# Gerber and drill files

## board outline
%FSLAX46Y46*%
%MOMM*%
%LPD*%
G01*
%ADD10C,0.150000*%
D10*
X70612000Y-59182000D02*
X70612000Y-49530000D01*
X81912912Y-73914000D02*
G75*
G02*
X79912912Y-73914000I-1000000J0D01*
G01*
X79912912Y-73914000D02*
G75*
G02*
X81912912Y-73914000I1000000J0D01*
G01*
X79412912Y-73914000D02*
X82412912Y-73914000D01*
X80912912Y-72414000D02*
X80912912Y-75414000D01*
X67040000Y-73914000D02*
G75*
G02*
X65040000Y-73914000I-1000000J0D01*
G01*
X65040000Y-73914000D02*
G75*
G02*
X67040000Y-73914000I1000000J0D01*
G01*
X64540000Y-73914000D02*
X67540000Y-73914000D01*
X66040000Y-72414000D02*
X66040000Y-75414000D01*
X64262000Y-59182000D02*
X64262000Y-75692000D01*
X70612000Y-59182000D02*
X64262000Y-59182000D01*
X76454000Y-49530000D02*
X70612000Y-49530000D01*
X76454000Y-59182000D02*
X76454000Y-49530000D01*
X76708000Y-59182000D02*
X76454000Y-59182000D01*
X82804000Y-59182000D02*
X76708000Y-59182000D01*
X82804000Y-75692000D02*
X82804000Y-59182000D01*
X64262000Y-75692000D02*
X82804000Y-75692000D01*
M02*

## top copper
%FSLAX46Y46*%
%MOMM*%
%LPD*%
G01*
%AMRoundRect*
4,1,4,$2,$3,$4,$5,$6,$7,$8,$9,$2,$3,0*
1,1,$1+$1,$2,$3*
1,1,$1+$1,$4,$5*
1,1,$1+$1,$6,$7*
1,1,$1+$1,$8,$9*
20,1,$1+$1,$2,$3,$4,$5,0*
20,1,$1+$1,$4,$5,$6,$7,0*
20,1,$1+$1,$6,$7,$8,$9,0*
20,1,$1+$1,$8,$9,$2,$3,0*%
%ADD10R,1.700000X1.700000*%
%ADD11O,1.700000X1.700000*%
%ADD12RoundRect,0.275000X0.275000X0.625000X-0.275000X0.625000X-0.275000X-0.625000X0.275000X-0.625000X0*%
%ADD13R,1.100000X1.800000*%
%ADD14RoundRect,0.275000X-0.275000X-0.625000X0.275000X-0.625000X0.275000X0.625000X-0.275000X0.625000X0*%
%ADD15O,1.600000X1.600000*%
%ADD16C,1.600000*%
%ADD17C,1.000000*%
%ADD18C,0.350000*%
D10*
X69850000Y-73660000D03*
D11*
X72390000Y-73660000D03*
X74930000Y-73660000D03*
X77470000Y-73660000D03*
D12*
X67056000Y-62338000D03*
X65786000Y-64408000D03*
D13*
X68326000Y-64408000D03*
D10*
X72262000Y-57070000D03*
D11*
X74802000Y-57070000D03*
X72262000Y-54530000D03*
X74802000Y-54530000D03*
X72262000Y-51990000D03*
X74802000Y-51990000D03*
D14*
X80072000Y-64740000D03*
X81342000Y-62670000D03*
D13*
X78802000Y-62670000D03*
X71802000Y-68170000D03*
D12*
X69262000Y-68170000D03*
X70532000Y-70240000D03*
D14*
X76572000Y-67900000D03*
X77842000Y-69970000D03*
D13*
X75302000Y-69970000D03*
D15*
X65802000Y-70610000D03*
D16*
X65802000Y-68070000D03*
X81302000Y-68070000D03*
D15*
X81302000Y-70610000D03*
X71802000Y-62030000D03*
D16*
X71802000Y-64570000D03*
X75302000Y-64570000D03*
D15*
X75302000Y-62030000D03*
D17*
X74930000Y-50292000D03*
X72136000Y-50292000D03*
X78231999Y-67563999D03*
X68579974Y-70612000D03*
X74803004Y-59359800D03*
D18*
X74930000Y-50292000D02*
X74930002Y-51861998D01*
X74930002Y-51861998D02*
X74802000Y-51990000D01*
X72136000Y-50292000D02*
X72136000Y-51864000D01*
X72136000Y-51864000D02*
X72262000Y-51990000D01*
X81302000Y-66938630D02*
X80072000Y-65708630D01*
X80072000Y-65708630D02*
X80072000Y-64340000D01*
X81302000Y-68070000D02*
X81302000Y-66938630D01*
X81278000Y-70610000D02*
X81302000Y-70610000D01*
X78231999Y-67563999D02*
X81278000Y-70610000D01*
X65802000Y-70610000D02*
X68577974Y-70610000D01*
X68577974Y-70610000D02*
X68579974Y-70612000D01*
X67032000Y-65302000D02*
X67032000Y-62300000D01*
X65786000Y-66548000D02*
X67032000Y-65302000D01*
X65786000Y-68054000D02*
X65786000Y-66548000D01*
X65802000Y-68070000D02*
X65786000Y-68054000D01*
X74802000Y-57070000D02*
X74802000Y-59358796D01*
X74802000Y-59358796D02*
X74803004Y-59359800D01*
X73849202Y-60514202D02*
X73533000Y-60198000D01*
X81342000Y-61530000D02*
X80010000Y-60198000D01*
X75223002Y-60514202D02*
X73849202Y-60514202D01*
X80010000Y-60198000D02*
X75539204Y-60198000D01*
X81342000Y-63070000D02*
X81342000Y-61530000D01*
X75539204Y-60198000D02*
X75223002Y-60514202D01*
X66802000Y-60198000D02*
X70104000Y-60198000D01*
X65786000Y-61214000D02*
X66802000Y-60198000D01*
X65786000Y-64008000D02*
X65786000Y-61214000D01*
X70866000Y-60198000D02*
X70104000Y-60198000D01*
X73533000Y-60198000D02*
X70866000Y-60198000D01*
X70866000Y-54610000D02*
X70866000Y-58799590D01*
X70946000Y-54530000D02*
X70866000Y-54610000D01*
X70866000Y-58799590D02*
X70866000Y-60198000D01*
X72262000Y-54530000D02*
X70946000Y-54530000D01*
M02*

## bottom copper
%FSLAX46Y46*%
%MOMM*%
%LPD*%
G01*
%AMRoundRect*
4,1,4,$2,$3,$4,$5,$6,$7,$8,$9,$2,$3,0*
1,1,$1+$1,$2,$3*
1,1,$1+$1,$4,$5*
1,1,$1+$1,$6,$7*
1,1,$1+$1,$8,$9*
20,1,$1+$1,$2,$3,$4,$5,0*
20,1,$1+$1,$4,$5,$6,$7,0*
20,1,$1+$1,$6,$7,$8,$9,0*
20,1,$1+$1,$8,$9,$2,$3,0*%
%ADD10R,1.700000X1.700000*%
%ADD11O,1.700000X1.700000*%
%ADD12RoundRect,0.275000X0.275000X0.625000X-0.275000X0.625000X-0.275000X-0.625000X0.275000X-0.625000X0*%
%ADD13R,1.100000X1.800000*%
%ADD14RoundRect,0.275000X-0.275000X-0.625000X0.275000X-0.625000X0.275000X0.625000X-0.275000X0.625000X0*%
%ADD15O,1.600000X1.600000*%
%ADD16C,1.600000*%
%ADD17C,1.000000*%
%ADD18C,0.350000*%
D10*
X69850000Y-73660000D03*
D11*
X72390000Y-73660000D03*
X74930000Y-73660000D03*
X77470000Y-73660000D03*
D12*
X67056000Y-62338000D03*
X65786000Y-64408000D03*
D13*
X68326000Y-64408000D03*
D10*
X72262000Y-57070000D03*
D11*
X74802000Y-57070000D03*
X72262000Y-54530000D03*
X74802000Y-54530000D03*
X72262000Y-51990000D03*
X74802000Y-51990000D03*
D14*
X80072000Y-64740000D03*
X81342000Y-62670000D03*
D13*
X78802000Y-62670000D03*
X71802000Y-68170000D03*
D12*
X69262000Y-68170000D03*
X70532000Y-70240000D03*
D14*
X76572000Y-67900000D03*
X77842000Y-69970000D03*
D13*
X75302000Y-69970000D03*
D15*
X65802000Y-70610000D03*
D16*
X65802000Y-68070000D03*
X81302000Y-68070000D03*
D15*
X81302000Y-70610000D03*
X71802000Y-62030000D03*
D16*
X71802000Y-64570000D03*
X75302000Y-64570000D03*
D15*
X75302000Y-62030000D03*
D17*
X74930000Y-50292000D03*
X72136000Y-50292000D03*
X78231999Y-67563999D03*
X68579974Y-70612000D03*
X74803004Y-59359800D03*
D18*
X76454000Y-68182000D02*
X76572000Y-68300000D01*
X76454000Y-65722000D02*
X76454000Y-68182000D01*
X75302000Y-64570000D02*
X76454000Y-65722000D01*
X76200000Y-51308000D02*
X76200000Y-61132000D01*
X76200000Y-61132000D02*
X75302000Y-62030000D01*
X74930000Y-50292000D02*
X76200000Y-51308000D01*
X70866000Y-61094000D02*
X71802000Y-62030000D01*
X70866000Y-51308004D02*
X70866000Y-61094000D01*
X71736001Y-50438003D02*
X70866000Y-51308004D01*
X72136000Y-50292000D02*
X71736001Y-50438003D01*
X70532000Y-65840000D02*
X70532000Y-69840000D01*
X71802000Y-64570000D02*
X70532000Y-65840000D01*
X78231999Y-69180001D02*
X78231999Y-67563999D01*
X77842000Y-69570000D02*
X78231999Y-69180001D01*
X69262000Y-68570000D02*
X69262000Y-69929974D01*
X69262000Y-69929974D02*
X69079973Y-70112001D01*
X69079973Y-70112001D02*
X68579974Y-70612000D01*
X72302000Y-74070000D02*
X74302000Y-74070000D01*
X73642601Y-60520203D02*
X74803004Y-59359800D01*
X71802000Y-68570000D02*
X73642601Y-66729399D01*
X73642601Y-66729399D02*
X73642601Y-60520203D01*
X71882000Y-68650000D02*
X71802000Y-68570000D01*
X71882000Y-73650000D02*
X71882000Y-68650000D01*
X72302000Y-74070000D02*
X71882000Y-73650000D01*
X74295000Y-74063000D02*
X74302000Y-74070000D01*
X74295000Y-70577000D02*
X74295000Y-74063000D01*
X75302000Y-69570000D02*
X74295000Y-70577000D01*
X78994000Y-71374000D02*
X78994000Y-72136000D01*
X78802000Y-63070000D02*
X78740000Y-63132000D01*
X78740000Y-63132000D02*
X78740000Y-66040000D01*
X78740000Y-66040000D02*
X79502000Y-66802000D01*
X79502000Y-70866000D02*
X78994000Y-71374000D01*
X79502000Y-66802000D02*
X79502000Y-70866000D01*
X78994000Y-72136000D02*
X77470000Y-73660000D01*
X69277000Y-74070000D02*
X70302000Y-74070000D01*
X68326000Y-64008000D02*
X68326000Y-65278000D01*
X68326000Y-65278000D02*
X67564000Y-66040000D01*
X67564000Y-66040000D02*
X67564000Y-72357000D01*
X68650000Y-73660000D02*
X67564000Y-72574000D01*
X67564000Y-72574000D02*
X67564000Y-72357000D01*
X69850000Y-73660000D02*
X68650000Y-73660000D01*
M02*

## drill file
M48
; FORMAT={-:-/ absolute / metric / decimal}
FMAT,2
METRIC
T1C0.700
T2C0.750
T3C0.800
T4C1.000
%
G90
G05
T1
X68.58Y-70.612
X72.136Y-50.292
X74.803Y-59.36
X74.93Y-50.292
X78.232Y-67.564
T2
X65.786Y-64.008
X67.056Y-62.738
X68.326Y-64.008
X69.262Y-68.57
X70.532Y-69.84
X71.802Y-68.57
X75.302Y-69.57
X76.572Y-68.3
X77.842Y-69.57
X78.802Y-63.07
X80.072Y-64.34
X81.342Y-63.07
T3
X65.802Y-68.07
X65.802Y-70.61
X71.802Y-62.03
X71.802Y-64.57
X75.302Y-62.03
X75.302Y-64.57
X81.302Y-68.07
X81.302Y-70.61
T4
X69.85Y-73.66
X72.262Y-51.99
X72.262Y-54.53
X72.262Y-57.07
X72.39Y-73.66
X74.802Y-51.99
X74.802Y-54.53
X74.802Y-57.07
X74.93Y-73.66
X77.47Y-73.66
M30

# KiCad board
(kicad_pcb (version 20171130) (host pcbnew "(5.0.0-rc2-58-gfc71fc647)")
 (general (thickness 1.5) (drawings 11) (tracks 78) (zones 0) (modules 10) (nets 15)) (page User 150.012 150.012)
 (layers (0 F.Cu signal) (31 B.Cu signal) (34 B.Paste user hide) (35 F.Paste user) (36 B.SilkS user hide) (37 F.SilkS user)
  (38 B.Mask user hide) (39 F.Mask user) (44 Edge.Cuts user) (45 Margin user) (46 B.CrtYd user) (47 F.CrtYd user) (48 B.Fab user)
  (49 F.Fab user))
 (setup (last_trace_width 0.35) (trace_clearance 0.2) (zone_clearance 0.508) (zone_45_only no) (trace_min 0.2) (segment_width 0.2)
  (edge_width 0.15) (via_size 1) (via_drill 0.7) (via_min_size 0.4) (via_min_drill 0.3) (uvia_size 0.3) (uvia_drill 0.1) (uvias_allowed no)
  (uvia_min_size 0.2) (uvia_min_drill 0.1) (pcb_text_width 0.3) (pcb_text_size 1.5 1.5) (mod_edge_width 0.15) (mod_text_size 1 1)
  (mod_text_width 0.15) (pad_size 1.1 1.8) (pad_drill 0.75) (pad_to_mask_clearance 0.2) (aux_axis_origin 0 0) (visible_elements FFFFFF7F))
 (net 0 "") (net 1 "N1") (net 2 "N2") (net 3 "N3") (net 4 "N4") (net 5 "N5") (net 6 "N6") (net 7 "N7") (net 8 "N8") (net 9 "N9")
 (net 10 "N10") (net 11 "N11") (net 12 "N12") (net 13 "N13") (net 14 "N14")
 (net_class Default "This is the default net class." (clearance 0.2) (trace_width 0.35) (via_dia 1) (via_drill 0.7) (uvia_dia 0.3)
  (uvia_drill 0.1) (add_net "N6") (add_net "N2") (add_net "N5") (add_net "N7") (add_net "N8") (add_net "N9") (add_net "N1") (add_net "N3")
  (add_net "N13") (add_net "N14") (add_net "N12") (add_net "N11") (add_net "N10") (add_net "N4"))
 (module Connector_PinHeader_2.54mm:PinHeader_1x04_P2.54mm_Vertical (layer F.Cu) (at 69.85 73.66 90)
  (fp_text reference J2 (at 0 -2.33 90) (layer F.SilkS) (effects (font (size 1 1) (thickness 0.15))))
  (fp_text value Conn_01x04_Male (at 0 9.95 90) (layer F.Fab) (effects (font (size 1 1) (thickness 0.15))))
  (pad 1 thru_hole rect (at 0 0 90) (size 1.7 1.7) (drill 1) (layers *.Cu *.Mask) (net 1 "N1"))
  (pad 2 thru_hole oval (at 0 2.54 90) (size 1.7 1.7) (drill 1) (layers *.Cu *.Mask) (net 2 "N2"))
  (pad 3 thru_hole oval (at 0 5.08 90) (size 1.7 1.7) (drill 1) (layers *.Cu *.Mask) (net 2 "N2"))
  (pad 4 thru_hole oval (at 0 7.62 90) (size 1.7 1.7) (drill 1) (layers *.Cu *.Mask) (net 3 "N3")))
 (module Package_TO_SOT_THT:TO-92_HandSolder (layer B.Cu) (at 68.326 64.008 180)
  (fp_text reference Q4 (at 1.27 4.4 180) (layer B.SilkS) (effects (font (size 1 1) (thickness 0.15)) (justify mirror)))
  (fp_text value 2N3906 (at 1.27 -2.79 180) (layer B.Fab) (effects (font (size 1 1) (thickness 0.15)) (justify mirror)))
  (pad 2 thru_hole roundrect (at 1.27 1.27 180) (size 1.1 1.8) (drill 0.75 (offset 0 0.4)) (layers *.Cu *.Mask) (roundrect_rratio 0.25)
   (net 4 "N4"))
  (pad 3 thru_hole roundrect (at 2.54 0 180) (size 1.1 1.8) (drill 0.75 (offset 0 -0.4)) (layers *.Cu *.Mask) (roundrect_rratio 0.25)
   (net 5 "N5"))
  (pad 1 thru_hole rect (at 0 0 180) (size 1.1 1.8) (drill 0.75 (offset 0 -0.4)) (layers *.Cu *.Mask) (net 1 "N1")))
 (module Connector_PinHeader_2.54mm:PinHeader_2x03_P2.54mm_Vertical (layer B.Cu) (at 72.262 57.07)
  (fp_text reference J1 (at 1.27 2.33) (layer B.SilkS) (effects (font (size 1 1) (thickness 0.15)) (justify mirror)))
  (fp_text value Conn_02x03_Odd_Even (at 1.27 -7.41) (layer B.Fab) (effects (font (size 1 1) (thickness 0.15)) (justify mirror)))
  (pad 1 thru_hole rect (at 0 0) (size 1.7 1.7) (drill 1) (layers *.Cu *.Mask) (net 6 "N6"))
  (pad 2 thru_hole oval (at 2.54 0) (size 1.7 1.7) (drill 1) (layers *.Cu *.Mask) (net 2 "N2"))
  (pad 3 thru_hole oval (at 0 -2.54) (size 1.7 1.7) (drill 1) (layers *.Cu *.Mask) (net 5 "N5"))
  (pad 4 thru_hole oval (at 2.54 -2.54) (size 1.7 1.7) (drill 1) (layers *.Cu *.Mask) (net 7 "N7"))
  (pad 5 thru_hole oval (at 0 -5.08) (size 1.7 1.7) (drill 1) (layers *.Cu *.Mask) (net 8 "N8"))
  (pad 6 thru_hole oval (at 2.54 -5.08) (size 1.7 1.7) (drill 1) (layers *.Cu *.Mask) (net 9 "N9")))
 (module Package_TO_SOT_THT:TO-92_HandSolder (layer B.Cu) (at 78.802 63.07)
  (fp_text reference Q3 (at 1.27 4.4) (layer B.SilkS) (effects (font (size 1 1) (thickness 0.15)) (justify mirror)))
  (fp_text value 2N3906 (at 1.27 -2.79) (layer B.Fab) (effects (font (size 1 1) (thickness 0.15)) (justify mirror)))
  (pad 2 thru_hole roundrect (at 1.27 1.27) (size 1.1 1.8) (drill 0.75 (offset 0 0.4)) (layers *.Cu *.Mask) (roundrect_rratio 0.25)
   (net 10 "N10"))
  (pad 3 thru_hole roundrect (at 2.54 0) (size 1.1 1.8) (drill 0.75 (offset 0 -0.4)) (layers *.Cu *.Mask) (roundrect_rratio 0.25)
   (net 5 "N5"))
  (pad 1 thru_hole rect (at 0 0) (size 1.1 1.8) (drill 0.75 (offset 0 -0.4)) (layers *.Cu *.Mask) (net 3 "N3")))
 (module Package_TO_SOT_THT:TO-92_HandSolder (layer F.Cu) (at 71.802 68.57 180)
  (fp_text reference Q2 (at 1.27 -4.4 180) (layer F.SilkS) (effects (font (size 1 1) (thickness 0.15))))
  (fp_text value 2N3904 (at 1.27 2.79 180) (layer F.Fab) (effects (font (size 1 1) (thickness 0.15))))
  (pad 1 thru_hole rect (at 0 0 180) (size 1.1 1.8) (drill 0.75 (offset 0 0.4)) (layers *.Cu *.Mask) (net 2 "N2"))
  (pad 3 thru_hole roundrect (at 2.54 0 180) (size 1.1 1.8) (drill 0.75 (offset 0 0.4)) (layers *.Cu *.Mask) (roundrect_rratio 0.25)
   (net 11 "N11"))
  (pad 2 thru_hole roundrect (at 1.27 -1.27 180) (size 1.1 1.8) (drill 0.75 (offset 0 -0.4)) (layers *.Cu *.Mask) (roundrect_rratio 0.25)
   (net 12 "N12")))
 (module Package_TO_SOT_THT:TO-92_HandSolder (layer F.Cu) (at 75.302 69.57)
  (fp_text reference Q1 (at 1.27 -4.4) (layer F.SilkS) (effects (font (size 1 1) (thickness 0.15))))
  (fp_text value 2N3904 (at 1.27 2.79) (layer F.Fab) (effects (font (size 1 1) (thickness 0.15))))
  (pad 2 thru_hole roundrect (at 1.27 -1.27) (size 1.1 1.8) (drill 0.75 (offset 0 -0.4)) (layers *.Cu *.Mask) (roundrect_rratio 0.25)
   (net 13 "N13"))
  (pad 3 thru_hole roundrect (at 2.54 0) (size 1.1 1.8) (drill 0.75 (offset 0 0.4)) (layers *.Cu *.Mask) (roundrect_rratio 0.25)
   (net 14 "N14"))
  (pad 1 thru_hole rect (at 0 0) (size 1.1 1.8) (drill 0.75 (offset 0 0.4)) (layers *.Cu *.Mask) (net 2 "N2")))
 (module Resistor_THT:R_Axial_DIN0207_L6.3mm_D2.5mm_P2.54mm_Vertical (layer B.Cu) (at 65.802 68.07 270)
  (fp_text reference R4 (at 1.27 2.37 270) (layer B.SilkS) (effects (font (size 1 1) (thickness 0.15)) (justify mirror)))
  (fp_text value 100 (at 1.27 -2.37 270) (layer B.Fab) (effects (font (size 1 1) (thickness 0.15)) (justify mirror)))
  (pad 2 thru_hole oval (at 2.54 0 270) (size 1.6 1.6) (drill 0.8) (layers *.Cu *.Mask) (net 11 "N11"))
  (pad 1 thru_hole circle (at 0 0 270) (size 1.6 1.6) (drill 0.8) (layers *.Cu *.Mask) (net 4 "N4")))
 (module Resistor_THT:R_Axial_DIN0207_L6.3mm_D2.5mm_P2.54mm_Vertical (layer B.Cu) (at 81.302 68.07 270)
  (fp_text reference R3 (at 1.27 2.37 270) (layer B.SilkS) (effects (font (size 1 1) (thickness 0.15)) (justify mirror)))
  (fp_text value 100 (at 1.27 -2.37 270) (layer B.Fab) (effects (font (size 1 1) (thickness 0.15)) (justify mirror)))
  (pad 1 thru_hole circle (at 0 0 270) (size 1.6 1.6) (drill 0.8) (layers *.Cu *.Mask) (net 10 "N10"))
  (pad 2 thru_hole oval (at 2.54 0 270) (size 1.6 1.6) (drill 0.8) (layers *.Cu *.Mask) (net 14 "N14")))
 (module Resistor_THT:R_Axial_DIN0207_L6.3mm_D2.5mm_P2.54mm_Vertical (layer F.Cu) (at 71.802 64.57 90)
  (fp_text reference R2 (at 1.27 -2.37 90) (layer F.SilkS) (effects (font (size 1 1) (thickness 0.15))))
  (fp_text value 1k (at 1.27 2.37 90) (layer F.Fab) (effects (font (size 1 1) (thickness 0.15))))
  (pad 2 thru_hole oval (at 2.54 0 90) (size 1.6 1.6) (drill 0.8) (layers *.Cu *.Mask) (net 8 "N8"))
  (pad 1 thru_hole circle (at 0 0 90) (size 1.6 1.6) (drill 0.8) (layers *.Cu *.Mask) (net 12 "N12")))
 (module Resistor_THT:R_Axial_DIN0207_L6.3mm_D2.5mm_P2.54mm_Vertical (layer F.Cu) (at 75.302 64.57 90)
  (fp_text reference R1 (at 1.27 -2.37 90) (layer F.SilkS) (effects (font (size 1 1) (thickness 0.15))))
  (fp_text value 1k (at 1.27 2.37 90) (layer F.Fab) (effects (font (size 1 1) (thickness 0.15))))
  (pad 1 thru_hole circle (at 0 0 90) (size 1.6 1.6) (drill 0.8) (layers *.Cu *.Mask) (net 13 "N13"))
  (pad 2 thru_hole oval (at 2.54 0 90) (size 1.6 1.6) (drill 0.8) (layers *.Cu *.Mask) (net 9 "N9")))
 (gr_line (start 70.612 59.182) (end 70.612 49.53) (layer Edge.Cuts) (width 0.15))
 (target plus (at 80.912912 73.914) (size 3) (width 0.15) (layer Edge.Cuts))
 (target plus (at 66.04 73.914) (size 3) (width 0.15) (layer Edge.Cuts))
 (gr_line (start 64.262 59.182) (end 64.262 75.692) (layer Edge.Cuts) (width 0.15))
 (gr_line (start 70.612 59.182) (end 64.262 59.182) (layer Edge.Cuts) (width 0.15))
 (gr_line (start 76.454 49.53) (end 70.612 49.53) (layer Edge.Cuts) (width 0.15))
 (gr_line (start 76.454 59.182) (end 76.454 49.53) (layer Edge.Cuts) (width 0.15))
 (gr_line (start 76.708 59.182) (end 76.454 59.182) (layer Edge.Cuts) (width 0.15))
 (gr_line (start 82.804 59.182) (end 76.708 59.182) (layer Edge.Cuts) (width 0.15))
 (gr_line (start 82.804 75.692) (end 82.804 59.182) (layer Edge.Cuts) (width 0.15))
 (gr_line (start 64.262 75.692) (end 82.804 75.692) (layer Edge.Cuts) (width 0.15))
 (segment (start 76.454 68.182) (end 76.572 68.3) (width 0.35) (layer B.Cu) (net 13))
 (segment (start 76.454 65.722) (end 76.454 68.182) (width 0.35) (layer B.Cu) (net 13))
 (segment (start 75.302 64.57) (end 76.454 65.722) (width 0.35) (layer B.Cu) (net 13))
 (via (at 74.93 50.292) (size 1) (drill 0.7) (layers F.Cu B.Cu) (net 9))
 (segment (start 74.93 50.292) (end 74.930002 51.861998) (width 0.35) (layer F.Cu) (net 9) (status 20))
 (segment (start 76.2 51.308) (end 76.2 61.132) (width 0.35) (layer B.Cu) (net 9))
 (segment (start 74.930002 51.861998) (end 74.802 51.99) (width 0.35) (layer F.Cu) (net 9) (status 30))
 (segment (start 76.2 61.132) (end 75.302 62.03) (width 0.35) (layer B.Cu) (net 9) (status 20))
 (segment (start 74.93 50.292) (end 76.2 51.308) (width 0.35) (layer B.Cu) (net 9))
 (via (at 72.136 50.292) (size 1) (drill 0.7) (layers F.Cu B.Cu) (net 8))
 (segment (start 72.136 50.292) (end 72.136 51.864) (width 0.35) (layer F.Cu) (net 8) (status 20))
 (segment (start 72.136 51.864) (end 72.262 51.99) (width 0.35) (layer F.Cu) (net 8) (status 30))
 (segment (start 70.866 61.094) (end 71.802 62.03) (width 0.35) (layer B.Cu) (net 8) (status 20))
 (segment (start 70.866 51.308004) (end 70.866 61.094) (width 0.35) (layer B.Cu) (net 8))
 (segment (start 71.736001 50.438003) (end 70.866 51.308004) (width 0.35) (layer B.Cu) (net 8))
 (segment (start 72.136 50.292) (end 71.736001 50.438003) (width 0.35) (layer B.Cu) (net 8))
 (segment (start 70.532 65.84) (end 70.532 69.84) (width 0.35) (layer B.Cu) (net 12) (status 20))
 (segment (start 71.802 64.57) (end 70.532 65.84) (width 0.35) (layer B.Cu) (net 12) (status 10))
 (segment (start 81.302 66.93863) (end 80.072 65.70863) (width 0.35) (layer F.Cu) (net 10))
 (segment (start 80.072 65.70863) (end 80.072 64.34) (width 0.35) (layer F.Cu) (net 10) (status 20))
 (segment (start 81.302 68.07) (end 81.302 66.93863) (width 0.35) (layer F.Cu) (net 10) (status 10))
 (via (at 78.231999 67.563999) (size 1) (drill 0.7) (layers F.Cu B.Cu) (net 14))
 (segment (start 78.231999 69.180001) (end 78.231999 67.563999) (width 0.35) (layer B.Cu) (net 14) (status 10))
 (segment (start 77.842 69.57) (end 78.231999 69.180001) (width 0.35) (layer B.Cu) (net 14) (status 30))
 (segment (start 81.278 70.61) (end 81.302 70.61) (width 0.35) (layer F.Cu) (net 14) (status 30))
 (segment (start 78.231999 67.563999) (end 81.278 70.61) (width 0.35) (layer F.Cu) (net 14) (status 20))
 (segment (start 69.262 68.57) (end 69.262 69.929974) (width 0.35) (layer B.Cu) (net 11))
 (via (at 68.579974 70.612) (size 1) (drill 0.7) (layers F.Cu B.Cu) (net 11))
 (segment (start 69.262 69.929974) (end 69.079973 70.112001) (width 0.35) (layer B.Cu) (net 11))
 (segment (start 65.802 70.61) (end 68.577974 70.61) (width 0.35) (layer F.Cu) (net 11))
 (segment (start 69.079973 70.112001) (end 68.579974 70.612) (width 0.35) (layer B.Cu) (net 11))
 (segment (start 68.577974 70.61) (end 68.579974 70.612) (width 0.35) (layer F.Cu) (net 11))
 (segment (start 67.032 65.302) (end 67.032 62.3) (width 0.35) (layer F.Cu) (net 4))
 (segment (start 65.786 66.548) (end 67.032 65.302) (width 0.35) (layer F.Cu) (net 4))
 (segment (start 65.786 68.054) (end 65.786 66.548) (width 0.35) (layer F.Cu) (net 4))
 (segment (start 65.802 68.07) (end 65.786 68.054) (width 0.35) (layer F.Cu) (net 4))
 (segment (start 72.302 74.07) (end 74.302 74.07) (width 0.35) (layer B.Cu) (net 2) (status 30))
 (segment (start 74.802 57.07) (end 74.802 59.358796) (width 0.35) (layer F.Cu) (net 2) (status 10))
 (segment (start 73.642601 60.520203) (end 74.803004 59.3598) (width 0.35) (layer B.Cu) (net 2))
 (segment (start 74.802 59.358796) (end 74.803004 59.3598) (width 0.35) (layer F.Cu) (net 2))
 (segment (start 71.802 68.57) (end 73.642601 66.729399) (width 0.35) (layer B.Cu) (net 2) (status 10))
 (segment (start 73.642601 66.729399) (end 73.642601 60.520203) (width 0.35) (layer B.Cu) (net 2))
 (via (at 74.803004 59.3598) (size 1) (drill 0.7) (layers F.Cu B.Cu) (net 2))
 (segment (start 71.882 68.65) (end 71.802 68.57) (width 0.35) (layer B.Cu) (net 2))
 (segment (start 71.882 73.65) (end 71.882 68.65) (width 0.35) (layer B.Cu) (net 2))
 (segment (start 72.302 74.07) (end 71.882 73.65) (width 0.35) (layer B.Cu) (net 2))
 (segment (start 74.295 74.063) (end 74.302 74.07) (width 0.35) (layer B.Cu) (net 2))
 (segment (start 74.295 70.577) (end 74.295 74.063) (width 0.35) (layer B.Cu) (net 2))
 (segment (start 75.302 69.57) (end 74.295 70.577) (width 0.35) (layer B.Cu) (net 2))
 (segment (start 73.849202 60.514202) (end 73.533 60.198) (width 0.35) (layer F.Cu) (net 5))
 (segment (start 81.342 61.53) (end 80.01 60.198) (width 0.35) (layer F.Cu) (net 5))
 (segment (start 75.223002 60.514202) (end 73.849202 60.514202) (width 0.35) (layer F.Cu) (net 5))
 (segment (start 80.01 60.198) (end 75.539204 60.198) (width 0.35) (layer F.Cu) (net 5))
 (segment (start 81.342 63.07) (end 81.342 61.53) (width 0.35) (layer F.Cu) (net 5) (status 10))
 (segment (start 75.539204 60.198) (end 75.223002 60.514202) (width 0.35) (layer F.Cu) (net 5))
 (segment (start 66.802 60.198) (end 70.104 60.198) (width 0.35) (layer F.Cu) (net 5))
 (segment (start 65.786 61.214) (end 66.802 60.198) (width 0.35) (layer F.Cu) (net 5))
 (segment (start 65.786 64.008) (end 65.786 61.214) (width 0.35) (layer F.Cu) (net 5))
 (segment (start 70.866 60.198) (end 70.104 60.198) (width 0.35) (layer F.Cu) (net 5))
 (segment (start 73.533 60.198) (end 70.866 60.198) (width 0.35) (layer F.Cu) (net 5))
 (segment (start 70.866 54.61) (end 70.866 58.79959) (width 0.35) (layer F.Cu) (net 5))
 (segment (start 70.946 54.53) (end 70.866 54.61) (width 0.35) (layer F.Cu) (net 5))
 (segment (start 70.866 58.79959) (end 70.866 60.198) (width 0.35) (layer F.Cu) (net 5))
 (segment (start 72.262 54.53) (end 70.946 54.53) (width 0.35) (layer F.Cu) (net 5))
 (segment (start 78.994 71.374) (end 78.994 72.136) (width 0.35) (layer B.Cu) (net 3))
 (segment (start 78.802 63.07) (end 78.74 63.132) (width 0.35) (layer B.Cu) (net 3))
 (segment (start 78.74 63.132) (end 78.74 66.04) (width 0.35) (layer B.Cu) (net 3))
 (segment (start 78.74 66.04) (end 79.502 66.802) (width 0.35) (layer B.Cu) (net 3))
 (segment (start 79.502 70.866) (end 78.994 71.374) (width 0.35) (layer B.Cu) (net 3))
 (segment (start 79.502 66.802) (end 79.502 70.866) (width 0.35) (layer B.Cu) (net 3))
 (segment (start 78.994 72.136) (end 77.47 73.66) (width 0.35) (layer B.Cu) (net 3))
 (segment (start 69.277 74.07) (end 70.302 74.07) (width 0.35) (layer B.Cu) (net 1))
 (segment (start 68.326 64.008) (end 68.326 65.278) (width 0.35) (layer B.Cu) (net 1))
 (segment (start 68.326 65.278) (end 67.564 66.04) (width 0.35) (layer B.Cu) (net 1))
 (segment (start 67.564 66.04) (end 67.564 72.357) (width 0.35) (layer B.Cu) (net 1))
 (segment (start 68.65 73.66) (end 67.564 72.574) (width 0.35) (layer B.Cu) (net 1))
 (segment (start 67.564 72.574) (end 67.564 72.357) (width 0.35) (layer B.Cu) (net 1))
 (segment (start 69.85 73.66) (end 68.65 73.66) (width 0.35) (layer B.Cu) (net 1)))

